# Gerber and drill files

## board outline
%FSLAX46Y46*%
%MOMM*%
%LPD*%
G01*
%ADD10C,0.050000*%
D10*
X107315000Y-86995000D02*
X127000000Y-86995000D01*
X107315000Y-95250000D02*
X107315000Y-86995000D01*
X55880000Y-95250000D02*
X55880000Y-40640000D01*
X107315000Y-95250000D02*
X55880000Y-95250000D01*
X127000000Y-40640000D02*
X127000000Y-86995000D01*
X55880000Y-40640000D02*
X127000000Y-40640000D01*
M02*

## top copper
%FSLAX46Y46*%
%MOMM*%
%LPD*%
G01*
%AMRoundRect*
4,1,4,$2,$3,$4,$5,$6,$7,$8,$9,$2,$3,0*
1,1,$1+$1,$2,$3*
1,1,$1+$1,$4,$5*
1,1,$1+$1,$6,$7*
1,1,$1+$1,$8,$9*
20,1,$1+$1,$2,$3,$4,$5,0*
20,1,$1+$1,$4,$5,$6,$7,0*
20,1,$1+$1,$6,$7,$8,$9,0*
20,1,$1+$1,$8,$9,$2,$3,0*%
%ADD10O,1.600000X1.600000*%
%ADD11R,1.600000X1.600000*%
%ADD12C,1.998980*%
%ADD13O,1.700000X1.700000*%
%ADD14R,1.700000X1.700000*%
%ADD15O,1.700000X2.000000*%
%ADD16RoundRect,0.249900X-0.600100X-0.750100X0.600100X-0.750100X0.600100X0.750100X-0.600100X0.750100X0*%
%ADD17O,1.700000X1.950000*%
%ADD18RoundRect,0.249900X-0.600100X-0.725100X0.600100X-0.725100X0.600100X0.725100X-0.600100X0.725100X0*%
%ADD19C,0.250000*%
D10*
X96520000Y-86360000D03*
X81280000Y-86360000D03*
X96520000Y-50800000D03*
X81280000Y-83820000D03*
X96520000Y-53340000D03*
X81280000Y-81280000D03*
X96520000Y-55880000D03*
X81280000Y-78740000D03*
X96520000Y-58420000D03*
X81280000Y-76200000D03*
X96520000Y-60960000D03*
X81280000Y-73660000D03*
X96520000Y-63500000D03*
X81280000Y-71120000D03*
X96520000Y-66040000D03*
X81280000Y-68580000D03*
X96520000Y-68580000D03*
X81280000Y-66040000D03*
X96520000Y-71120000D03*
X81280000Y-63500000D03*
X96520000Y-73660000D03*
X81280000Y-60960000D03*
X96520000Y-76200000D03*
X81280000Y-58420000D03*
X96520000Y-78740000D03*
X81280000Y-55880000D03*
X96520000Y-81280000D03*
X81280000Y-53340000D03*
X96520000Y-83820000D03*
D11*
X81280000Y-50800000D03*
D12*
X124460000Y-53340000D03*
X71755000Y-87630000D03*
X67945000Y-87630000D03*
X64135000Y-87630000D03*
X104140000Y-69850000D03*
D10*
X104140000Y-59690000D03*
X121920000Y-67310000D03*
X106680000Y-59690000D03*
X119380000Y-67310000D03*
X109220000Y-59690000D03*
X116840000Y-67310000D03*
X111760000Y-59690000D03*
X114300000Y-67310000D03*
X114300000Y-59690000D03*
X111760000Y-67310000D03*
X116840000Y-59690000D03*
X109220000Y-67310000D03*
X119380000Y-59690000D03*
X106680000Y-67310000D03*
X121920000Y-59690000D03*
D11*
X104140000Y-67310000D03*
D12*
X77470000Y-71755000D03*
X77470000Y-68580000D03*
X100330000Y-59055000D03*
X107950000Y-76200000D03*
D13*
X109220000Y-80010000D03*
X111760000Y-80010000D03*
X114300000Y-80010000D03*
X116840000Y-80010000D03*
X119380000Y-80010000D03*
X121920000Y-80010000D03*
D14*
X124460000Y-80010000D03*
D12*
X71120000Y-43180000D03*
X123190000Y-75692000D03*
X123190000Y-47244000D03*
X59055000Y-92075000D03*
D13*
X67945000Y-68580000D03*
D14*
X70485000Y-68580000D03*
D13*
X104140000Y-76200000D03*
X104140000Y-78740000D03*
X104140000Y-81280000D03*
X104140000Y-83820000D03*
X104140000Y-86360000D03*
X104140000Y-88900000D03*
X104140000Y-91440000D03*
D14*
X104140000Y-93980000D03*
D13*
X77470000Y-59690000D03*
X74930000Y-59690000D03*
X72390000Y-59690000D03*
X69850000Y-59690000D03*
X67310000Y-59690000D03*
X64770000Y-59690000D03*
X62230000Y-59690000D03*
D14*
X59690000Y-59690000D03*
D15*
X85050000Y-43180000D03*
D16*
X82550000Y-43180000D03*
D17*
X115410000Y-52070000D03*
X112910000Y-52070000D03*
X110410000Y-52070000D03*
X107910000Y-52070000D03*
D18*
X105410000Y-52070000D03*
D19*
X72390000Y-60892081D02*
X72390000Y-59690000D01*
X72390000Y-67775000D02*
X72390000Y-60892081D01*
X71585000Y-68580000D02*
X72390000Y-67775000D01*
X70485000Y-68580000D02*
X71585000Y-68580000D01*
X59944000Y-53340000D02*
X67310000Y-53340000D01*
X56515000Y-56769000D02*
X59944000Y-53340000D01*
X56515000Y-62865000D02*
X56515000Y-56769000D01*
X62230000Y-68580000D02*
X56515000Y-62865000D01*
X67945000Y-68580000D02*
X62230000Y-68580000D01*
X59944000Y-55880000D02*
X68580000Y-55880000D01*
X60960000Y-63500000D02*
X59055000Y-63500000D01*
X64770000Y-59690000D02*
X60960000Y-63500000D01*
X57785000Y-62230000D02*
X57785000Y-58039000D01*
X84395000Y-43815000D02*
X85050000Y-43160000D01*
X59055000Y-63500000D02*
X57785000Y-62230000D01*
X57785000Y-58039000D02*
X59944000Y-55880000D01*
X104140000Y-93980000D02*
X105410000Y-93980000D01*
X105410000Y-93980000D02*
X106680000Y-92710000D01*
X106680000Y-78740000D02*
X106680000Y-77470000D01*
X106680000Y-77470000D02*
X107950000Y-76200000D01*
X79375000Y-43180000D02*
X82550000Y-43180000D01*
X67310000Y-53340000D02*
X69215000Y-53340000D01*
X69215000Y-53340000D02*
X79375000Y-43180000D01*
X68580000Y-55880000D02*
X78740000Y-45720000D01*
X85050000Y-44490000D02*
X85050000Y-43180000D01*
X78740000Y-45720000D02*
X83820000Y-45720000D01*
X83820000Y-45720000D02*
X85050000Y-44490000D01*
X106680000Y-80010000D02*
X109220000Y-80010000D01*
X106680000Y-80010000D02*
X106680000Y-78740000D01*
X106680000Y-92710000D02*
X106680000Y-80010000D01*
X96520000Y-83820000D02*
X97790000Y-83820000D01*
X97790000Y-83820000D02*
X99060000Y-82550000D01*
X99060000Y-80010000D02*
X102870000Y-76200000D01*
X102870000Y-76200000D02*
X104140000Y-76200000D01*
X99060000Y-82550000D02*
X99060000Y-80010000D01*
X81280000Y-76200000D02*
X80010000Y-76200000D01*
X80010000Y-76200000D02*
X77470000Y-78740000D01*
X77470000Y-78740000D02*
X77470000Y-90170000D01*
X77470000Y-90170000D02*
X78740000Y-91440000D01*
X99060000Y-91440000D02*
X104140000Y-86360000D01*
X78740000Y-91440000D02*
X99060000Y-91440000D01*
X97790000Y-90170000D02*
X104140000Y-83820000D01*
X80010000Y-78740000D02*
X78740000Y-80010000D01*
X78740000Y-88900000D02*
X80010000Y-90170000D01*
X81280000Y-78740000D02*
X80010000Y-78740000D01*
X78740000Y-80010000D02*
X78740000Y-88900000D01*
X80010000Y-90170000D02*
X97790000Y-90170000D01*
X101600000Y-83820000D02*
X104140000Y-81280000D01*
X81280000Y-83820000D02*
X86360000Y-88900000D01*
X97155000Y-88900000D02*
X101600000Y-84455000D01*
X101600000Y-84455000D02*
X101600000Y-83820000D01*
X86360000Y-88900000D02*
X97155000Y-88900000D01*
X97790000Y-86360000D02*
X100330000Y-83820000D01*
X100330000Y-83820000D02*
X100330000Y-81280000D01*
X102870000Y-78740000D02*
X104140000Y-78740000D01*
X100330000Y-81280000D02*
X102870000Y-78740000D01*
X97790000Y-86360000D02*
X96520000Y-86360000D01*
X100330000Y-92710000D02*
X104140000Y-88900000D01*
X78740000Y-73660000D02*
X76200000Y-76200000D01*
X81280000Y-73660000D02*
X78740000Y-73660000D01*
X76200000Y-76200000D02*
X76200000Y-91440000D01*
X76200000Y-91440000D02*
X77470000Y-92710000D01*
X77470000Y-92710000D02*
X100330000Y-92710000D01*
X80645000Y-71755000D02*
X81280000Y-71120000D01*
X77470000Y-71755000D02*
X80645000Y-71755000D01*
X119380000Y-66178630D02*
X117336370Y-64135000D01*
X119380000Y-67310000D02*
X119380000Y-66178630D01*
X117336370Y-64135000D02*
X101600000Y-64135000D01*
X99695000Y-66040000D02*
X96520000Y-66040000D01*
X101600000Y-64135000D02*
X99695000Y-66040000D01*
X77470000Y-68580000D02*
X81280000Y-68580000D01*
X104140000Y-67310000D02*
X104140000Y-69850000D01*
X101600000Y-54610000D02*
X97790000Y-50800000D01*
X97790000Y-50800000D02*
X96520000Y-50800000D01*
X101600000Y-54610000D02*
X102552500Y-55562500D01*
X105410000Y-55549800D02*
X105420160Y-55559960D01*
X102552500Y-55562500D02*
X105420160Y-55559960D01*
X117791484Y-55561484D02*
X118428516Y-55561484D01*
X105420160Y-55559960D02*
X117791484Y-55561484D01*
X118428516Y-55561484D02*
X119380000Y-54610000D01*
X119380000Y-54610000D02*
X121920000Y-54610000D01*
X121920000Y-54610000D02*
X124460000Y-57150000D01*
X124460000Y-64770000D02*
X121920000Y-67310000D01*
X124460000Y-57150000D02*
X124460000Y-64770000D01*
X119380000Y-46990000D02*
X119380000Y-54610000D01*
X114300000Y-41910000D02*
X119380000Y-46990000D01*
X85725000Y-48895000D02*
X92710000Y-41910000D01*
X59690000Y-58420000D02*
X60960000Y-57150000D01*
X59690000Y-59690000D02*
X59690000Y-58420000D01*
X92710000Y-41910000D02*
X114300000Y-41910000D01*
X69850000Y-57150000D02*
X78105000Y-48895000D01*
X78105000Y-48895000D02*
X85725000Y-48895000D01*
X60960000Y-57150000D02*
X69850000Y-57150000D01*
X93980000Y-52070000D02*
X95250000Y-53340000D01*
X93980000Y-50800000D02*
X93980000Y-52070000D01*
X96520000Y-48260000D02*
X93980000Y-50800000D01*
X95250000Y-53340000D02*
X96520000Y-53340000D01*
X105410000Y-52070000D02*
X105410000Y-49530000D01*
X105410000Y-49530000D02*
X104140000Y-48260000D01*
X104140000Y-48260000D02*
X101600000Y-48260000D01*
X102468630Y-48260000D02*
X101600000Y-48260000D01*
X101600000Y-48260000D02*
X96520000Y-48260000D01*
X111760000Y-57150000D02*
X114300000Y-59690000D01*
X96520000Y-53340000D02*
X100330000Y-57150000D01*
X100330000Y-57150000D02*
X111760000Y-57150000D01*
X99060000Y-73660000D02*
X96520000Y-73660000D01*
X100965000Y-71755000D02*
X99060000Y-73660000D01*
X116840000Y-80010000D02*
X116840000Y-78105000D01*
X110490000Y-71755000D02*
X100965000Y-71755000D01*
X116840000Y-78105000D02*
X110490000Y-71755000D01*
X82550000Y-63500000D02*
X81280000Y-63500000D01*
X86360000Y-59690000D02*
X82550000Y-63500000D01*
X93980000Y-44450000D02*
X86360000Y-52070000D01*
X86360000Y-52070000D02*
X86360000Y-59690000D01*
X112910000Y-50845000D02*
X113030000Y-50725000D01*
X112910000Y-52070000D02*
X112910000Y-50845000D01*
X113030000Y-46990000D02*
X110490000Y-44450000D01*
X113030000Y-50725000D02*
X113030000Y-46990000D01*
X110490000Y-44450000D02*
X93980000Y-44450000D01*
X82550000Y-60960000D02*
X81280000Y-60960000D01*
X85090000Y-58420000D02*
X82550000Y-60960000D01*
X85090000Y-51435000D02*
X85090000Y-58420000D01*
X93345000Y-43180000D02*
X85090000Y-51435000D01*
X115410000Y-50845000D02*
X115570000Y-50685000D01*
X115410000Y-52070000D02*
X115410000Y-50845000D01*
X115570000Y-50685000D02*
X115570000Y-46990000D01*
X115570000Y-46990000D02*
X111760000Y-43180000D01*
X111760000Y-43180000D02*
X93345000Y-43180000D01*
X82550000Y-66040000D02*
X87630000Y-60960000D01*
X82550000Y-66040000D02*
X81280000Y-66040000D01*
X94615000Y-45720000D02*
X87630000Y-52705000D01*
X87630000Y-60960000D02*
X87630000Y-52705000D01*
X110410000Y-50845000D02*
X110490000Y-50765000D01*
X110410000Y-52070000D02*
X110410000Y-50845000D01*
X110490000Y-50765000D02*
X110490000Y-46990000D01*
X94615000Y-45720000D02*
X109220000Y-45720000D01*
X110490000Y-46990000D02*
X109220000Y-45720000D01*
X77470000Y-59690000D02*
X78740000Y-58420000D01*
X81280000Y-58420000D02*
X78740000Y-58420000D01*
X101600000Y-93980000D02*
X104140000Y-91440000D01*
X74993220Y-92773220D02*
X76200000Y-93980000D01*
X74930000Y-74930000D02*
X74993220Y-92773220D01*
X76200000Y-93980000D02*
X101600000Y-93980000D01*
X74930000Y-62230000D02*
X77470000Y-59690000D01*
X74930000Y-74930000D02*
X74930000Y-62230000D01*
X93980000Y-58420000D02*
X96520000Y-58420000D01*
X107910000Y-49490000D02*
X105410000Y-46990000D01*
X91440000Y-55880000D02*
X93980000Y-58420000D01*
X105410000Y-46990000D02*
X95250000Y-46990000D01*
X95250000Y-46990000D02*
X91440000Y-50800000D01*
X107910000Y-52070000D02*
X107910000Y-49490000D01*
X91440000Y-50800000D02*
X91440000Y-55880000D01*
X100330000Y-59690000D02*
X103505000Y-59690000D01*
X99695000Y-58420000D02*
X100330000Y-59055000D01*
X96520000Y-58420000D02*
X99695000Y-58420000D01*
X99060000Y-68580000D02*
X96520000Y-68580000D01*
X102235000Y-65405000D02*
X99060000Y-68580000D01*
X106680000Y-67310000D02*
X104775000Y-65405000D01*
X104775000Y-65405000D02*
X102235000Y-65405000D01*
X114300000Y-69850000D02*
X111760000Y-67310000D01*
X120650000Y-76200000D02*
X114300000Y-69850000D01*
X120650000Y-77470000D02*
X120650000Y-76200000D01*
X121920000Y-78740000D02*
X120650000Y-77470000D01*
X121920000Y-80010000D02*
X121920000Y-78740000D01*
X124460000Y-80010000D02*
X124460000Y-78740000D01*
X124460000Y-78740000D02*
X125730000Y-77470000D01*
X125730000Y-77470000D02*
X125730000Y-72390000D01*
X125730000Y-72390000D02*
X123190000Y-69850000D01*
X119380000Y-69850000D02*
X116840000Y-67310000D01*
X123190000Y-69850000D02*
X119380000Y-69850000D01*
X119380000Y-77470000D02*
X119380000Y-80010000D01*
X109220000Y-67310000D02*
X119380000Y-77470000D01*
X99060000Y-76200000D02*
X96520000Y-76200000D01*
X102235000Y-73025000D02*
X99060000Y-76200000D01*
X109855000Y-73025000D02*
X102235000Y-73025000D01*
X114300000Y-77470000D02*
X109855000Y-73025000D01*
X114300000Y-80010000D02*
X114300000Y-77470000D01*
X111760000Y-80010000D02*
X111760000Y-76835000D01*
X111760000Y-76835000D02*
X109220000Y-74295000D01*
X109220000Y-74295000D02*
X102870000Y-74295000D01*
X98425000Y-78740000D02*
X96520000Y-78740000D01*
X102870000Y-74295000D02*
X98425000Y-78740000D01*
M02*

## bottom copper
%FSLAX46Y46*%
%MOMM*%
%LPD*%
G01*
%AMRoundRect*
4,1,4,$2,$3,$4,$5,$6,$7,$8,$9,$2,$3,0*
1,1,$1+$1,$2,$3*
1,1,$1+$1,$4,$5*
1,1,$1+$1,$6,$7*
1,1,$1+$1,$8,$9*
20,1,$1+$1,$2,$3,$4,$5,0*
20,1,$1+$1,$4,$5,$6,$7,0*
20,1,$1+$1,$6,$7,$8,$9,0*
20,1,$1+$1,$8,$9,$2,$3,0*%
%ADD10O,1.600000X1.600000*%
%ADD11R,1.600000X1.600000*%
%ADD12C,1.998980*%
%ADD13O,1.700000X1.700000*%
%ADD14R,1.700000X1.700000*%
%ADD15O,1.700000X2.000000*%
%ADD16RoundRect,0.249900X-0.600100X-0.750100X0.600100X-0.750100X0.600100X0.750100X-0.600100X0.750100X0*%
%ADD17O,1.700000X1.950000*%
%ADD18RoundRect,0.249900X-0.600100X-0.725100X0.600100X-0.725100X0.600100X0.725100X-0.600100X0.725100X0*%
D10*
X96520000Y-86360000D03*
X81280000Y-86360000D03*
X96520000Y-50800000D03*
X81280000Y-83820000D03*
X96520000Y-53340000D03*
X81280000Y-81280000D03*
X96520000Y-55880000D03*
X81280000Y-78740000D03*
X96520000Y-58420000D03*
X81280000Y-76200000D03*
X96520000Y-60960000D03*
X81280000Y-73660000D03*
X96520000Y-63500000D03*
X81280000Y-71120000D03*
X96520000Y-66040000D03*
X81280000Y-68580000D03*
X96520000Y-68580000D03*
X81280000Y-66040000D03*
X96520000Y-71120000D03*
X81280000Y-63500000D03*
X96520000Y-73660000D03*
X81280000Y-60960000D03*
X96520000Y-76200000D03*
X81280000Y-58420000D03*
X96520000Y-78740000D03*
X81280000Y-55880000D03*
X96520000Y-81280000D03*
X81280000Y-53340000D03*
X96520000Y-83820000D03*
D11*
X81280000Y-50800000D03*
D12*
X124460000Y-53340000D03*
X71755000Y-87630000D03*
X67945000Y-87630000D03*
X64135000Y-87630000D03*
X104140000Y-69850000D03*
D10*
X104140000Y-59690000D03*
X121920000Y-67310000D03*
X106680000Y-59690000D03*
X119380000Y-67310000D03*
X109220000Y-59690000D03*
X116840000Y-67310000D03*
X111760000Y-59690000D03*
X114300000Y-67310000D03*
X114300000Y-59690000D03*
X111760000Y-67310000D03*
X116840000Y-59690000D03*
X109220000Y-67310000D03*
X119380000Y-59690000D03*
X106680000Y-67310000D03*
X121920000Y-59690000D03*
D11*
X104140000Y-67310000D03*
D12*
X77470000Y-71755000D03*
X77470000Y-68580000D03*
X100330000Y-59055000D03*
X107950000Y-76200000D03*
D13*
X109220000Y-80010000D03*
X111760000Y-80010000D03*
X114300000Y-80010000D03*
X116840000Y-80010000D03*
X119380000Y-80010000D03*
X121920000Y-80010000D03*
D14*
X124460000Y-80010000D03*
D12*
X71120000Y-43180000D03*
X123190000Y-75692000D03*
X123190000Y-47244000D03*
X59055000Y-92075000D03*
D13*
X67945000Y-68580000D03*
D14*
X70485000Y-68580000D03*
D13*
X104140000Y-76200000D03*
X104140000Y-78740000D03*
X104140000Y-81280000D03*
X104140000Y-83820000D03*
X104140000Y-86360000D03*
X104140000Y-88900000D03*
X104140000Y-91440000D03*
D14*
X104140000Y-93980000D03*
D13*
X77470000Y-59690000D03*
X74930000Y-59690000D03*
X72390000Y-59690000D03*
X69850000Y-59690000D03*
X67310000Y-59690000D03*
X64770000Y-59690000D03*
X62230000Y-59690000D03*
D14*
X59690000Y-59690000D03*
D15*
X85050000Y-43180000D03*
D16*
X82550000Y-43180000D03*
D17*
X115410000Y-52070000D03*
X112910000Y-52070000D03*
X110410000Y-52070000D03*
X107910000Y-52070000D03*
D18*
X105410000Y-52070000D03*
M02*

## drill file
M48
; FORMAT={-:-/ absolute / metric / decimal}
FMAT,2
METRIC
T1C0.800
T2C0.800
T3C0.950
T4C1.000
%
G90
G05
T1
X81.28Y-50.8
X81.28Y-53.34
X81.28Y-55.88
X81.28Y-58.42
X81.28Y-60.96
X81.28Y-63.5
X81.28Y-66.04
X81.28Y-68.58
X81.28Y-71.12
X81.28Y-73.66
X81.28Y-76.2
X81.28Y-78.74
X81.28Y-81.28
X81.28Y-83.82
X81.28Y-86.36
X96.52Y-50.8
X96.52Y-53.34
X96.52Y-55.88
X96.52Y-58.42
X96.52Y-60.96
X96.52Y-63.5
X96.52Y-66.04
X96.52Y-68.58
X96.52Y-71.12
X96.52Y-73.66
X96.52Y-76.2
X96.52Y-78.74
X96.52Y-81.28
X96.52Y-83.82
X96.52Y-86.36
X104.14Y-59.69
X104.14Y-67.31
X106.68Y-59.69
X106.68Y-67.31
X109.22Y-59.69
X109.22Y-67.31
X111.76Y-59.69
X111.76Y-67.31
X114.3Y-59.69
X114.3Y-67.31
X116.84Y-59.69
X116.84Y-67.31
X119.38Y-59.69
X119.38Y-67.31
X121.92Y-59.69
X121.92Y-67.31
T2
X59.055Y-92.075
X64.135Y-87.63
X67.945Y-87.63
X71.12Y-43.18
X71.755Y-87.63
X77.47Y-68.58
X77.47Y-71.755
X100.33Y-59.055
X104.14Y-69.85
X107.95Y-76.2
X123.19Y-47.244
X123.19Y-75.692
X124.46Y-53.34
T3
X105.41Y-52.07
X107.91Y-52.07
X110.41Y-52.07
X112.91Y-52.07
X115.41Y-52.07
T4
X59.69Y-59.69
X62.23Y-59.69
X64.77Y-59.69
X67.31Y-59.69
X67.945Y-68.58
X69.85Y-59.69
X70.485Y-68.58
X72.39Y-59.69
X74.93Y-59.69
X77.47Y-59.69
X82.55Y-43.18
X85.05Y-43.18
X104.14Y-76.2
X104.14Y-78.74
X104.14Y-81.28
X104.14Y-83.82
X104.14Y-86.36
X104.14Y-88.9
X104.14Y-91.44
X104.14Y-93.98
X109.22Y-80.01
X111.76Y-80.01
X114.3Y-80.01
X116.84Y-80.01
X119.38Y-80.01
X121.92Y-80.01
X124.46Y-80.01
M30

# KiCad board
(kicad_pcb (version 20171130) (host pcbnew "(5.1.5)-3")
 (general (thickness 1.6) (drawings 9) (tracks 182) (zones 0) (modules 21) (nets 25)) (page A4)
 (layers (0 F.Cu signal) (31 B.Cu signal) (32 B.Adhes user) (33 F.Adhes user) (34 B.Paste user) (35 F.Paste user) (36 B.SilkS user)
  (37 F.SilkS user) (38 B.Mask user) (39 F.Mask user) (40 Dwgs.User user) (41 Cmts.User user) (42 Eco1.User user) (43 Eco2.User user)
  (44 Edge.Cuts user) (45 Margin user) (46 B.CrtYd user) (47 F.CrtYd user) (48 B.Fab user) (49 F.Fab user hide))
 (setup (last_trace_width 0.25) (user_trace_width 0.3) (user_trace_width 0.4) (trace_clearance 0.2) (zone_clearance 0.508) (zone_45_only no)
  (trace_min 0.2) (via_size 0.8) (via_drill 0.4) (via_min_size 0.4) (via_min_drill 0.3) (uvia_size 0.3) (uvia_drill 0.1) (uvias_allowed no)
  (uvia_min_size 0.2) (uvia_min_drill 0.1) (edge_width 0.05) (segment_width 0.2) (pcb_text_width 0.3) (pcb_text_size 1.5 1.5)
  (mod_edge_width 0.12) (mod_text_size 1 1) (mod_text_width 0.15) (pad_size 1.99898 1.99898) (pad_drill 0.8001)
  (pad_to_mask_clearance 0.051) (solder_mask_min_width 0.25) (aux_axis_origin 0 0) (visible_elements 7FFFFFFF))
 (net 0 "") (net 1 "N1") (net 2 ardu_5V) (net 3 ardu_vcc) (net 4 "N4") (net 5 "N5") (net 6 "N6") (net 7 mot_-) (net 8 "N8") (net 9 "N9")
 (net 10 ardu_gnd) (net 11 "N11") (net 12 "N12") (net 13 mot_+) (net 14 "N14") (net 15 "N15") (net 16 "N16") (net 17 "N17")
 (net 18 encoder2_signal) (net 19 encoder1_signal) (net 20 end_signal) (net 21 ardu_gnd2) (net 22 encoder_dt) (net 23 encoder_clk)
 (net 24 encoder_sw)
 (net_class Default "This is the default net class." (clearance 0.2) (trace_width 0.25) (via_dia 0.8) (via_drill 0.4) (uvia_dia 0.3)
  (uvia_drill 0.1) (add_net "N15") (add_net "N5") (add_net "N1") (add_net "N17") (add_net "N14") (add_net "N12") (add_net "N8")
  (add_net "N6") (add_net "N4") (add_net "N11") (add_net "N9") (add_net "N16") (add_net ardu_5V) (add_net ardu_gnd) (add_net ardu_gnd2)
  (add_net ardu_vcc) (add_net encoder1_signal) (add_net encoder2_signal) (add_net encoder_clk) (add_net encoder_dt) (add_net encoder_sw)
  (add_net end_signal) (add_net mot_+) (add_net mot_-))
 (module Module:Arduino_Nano (layer F.Cu) (at 81.28 50.8)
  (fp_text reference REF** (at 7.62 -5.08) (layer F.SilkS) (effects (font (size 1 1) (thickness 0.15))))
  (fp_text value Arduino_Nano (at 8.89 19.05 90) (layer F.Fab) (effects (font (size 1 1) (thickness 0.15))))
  (pad 16 thru_hole oval (at 15.24 35.56) (size 1.6 1.6) (drill 0.8) (layers *.Cu *.Mask))
  (pad 15 thru_hole oval (at 0 35.56) (size 1.6 1.6) (drill 0.8) (layers *.Cu *.Mask))
  (pad 30 thru_hole oval (at 15.24 0) (size 1.6 1.6) (drill 0.8) (layers *.Cu *.Mask))
  (pad 14 thru_hole oval (at 0 33.02) (size 1.6 1.6) (drill 0.8) (layers *.Cu *.Mask))
  (pad 29 thru_hole oval (at 15.24 2.54) (size 1.6 1.6) (drill 0.8) (layers *.Cu *.Mask))
  (pad 13 thru_hole oval (at 0 30.48) (size 1.6 1.6) (drill 0.8) (layers *.Cu *.Mask))
  (pad 28 thru_hole oval (at 15.24 5.08) (size 1.6 1.6) (drill 0.8) (layers *.Cu *.Mask))
  (pad 12 thru_hole oval (at 0 27.94) (size 1.6 1.6) (drill 0.8) (layers *.Cu *.Mask))
  (pad 27 thru_hole oval (at 15.24 7.62) (size 1.6 1.6) (drill 0.8) (layers *.Cu *.Mask))
  (pad 11 thru_hole oval (at 0 25.4) (size 1.6 1.6) (drill 0.8) (layers *.Cu *.Mask))
  (pad 26 thru_hole oval (at 15.24 10.16) (size 1.6 1.6) (drill 0.8) (layers *.Cu *.Mask))
  (pad 10 thru_hole oval (at 0 22.86) (size 1.6 1.6) (drill 0.8) (layers *.Cu *.Mask))
  (pad 25 thru_hole oval (at 15.24 12.7) (size 1.6 1.6) (drill 0.8) (layers *.Cu *.Mask))
  (pad 9 thru_hole oval (at 0 20.32) (size 1.6 1.6) (drill 0.8) (layers *.Cu *.Mask))
  (pad 24 thru_hole oval (at 15.24 15.24) (size 1.6 1.6) (drill 0.8) (layers *.Cu *.Mask))
  (pad 8 thru_hole oval (at 0 17.78) (size 1.6 1.6) (drill 0.8) (layers *.Cu *.Mask))
  (pad 23 thru_hole oval (at 15.24 17.78) (size 1.6 1.6) (drill 0.8) (layers *.Cu *.Mask))
  (pad 7 thru_hole oval (at 0 15.24) (size 1.6 1.6) (drill 0.8) (layers *.Cu *.Mask))
  (pad 22 thru_hole oval (at 15.24 20.32) (size 1.6 1.6) (drill 0.8) (layers *.Cu *.Mask))
  (pad 6 thru_hole oval (at 0 12.7) (size 1.6 1.6) (drill 0.8) (layers *.Cu *.Mask))
  (pad 21 thru_hole oval (at 15.24 22.86) (size 1.6 1.6) (drill 0.8) (layers *.Cu *.Mask))
  (pad 5 thru_hole oval (at 0 10.16) (size 1.6 1.6) (drill 0.8) (layers *.Cu *.Mask))
  (pad 20 thru_hole oval (at 15.24 25.4) (size 1.6 1.6) (drill 0.8) (layers *.Cu *.Mask))
  (pad 4 thru_hole oval (at 0 7.62) (size 1.6 1.6) (drill 0.8) (layers *.Cu *.Mask))
  (pad 19 thru_hole oval (at 15.24 27.94) (size 1.6 1.6) (drill 0.8) (layers *.Cu *.Mask))
  (pad 3 thru_hole oval (at 0 5.08) (size 1.6 1.6) (drill 0.8) (layers *.Cu *.Mask))
  (pad 18 thru_hole oval (at 15.24 30.48) (size 1.6 1.6) (drill 0.8) (layers *.Cu *.Mask))
  (pad 2 thru_hole oval (at 0 2.54) (size 1.6 1.6) (drill 0.8) (layers *.Cu *.Mask))
  (pad 17 thru_hole oval (at 15.24 33.02) (size 1.6 1.6) (drill 0.8) (layers *.Cu *.Mask))
  (pad 1 thru_hole rect (at 0 0) (size 1.6 1.6) (drill 0.8) (layers *.Cu *.Mask)))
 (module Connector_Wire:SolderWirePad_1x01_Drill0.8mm (layer F.Cu) (at 124.46 53.34)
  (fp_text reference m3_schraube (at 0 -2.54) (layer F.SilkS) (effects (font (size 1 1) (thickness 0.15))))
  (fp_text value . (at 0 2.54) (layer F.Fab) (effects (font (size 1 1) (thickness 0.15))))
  (pad 1 thru_hole circle (at 0 0) (size 1.99898 1.99898) (drill 0.8001) (layers *.Cu *.Mask)))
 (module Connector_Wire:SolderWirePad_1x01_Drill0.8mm (layer F.Cu) (at 71.755 87.63)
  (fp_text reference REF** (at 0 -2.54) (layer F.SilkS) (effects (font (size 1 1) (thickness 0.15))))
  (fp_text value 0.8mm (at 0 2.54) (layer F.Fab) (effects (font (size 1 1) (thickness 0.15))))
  (pad 1 thru_hole circle (at 0 0) (size 1.99898 1.99898) (drill 0.8001) (layers *.Cu *.Mask)))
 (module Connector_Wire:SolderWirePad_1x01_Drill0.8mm (layer F.Cu) (at 67.945 87.63)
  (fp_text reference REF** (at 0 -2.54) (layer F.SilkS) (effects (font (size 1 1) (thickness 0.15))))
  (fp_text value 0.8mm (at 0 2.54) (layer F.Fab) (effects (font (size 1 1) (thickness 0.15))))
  (pad 1 thru_hole circle (at 0 0) (size 1.99898 1.99898) (drill 0.8001) (layers *.Cu *.Mask)))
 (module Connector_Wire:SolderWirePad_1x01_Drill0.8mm (layer F.Cu) (at 64.135 87.63)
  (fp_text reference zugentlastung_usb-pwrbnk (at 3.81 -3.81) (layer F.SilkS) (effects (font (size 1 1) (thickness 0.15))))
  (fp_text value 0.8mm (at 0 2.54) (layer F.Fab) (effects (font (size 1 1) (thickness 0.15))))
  (pad 1 thru_hole circle (at 0 0) (size 1.99898 1.99898) (drill 0.8001) (layers *.Cu *.Mask)))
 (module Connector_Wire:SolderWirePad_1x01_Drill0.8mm (layer F.Cu) (at 104.14 69.85)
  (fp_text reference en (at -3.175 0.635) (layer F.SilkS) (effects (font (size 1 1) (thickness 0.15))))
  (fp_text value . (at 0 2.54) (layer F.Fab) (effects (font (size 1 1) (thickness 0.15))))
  (pad 1 thru_hole circle (at 0 0) (size 1.99898 1.99898) (drill 0.8001) (layers *.Cu *.Mask) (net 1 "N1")))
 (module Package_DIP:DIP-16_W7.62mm (layer F.Cu) (at 104.14 67.31 90)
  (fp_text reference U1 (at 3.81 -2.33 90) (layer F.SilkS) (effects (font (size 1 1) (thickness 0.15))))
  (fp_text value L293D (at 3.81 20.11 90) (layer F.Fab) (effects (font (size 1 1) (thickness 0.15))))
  (pad 16 thru_hole oval (at 7.62 0 90) (size 1.6 1.6) (drill 0.8) (layers *.Cu *.Mask) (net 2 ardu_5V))
  (pad 8 thru_hole oval (at 0 17.78 90) (size 1.6 1.6) (drill 0.8) (layers *.Cu *.Mask) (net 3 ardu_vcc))
  (pad 15 thru_hole oval (at 7.62 2.54 90) (size 1.6 1.6) (drill 0.8) (layers *.Cu *.Mask) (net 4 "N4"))
  (pad 7 thru_hole oval (at 0 15.24 90) (size 1.6 1.6) (drill 0.8) (layers *.Cu *.Mask) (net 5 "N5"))
  (pad 14 thru_hole oval (at 7.62 5.08 90) (size 1.6 1.6) (drill 0.8) (layers *.Cu *.Mask) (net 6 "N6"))
  (pad 6 thru_hole oval (at 0 12.7 90) (size 1.6 1.6) (drill 0.8) (layers *.Cu *.Mask) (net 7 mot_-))
  (pad 13 thru_hole oval (at 7.62 7.62 90) (size 1.6 1.6) (drill 0.8) (layers *.Cu *.Mask) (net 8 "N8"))
  (pad 5 thru_hole oval (at 0 10.16 90) (size 1.6 1.6) (drill 0.8) (layers *.Cu *.Mask) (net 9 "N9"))
  (pad 12 thru_hole oval (at 7.62 10.16 90) (size 1.6 1.6) (drill 0.8) (layers *.Cu *.Mask) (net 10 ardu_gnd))
  (pad 4 thru_hole oval (at 0 7.62 90) (size 1.6 1.6) (drill 0.8) (layers *.Cu *.Mask) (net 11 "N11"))
  (pad 11 thru_hole oval (at 7.62 12.7 90) (size 1.6 1.6) (drill 0.8) (layers *.Cu *.Mask) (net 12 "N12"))
  (pad 3 thru_hole oval (at 0 5.08 90) (size 1.6 1.6) (drill 0.8) (layers *.Cu *.Mask) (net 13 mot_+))
  (pad 10 thru_hole oval (at 7.62 15.24 90) (size 1.6 1.6) (drill 0.8) (layers *.Cu *.Mask) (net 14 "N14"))
  (pad 2 thru_hole oval (at 0 2.54 90) (size 1.6 1.6) (drill 0.8) (layers *.Cu *.Mask) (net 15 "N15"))
  (pad 9 thru_hole oval (at 7.62 17.78 90) (size 1.6 1.6) (drill 0.8) (layers *.Cu *.Mask) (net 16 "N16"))
  (pad 1 thru_hole rect (at 0 0 90) (size 1.6 1.6) (drill 0.8) (layers *.Cu *.Mask) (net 1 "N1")))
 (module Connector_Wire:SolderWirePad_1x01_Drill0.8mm (layer F.Cu) (at 77.47 71.755)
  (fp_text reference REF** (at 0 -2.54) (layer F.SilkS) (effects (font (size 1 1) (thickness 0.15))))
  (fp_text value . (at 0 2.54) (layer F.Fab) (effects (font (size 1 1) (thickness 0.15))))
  (pad 1 thru_hole circle (at 0 0) (size 1.99898 1.99898) (drill 0.8001) (layers *.Cu *.Mask) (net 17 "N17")))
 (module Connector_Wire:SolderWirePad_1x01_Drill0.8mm (layer F.Cu) (at 77.47 68.58)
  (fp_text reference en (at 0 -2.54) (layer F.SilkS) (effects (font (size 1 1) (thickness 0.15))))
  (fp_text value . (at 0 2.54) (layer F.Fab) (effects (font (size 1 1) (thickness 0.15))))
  (pad 1 thru_hole circle (at 0 0) (size 1.99898 1.99898) (drill 0.8001) (layers *.Cu *.Mask) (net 1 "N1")))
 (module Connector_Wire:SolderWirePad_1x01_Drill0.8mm (layer F.Cu) (at 100.33 59.055)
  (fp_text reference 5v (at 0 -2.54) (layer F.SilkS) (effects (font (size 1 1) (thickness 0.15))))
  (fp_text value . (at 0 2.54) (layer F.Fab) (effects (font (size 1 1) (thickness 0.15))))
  (pad 1 thru_hole circle (at 0 0) (size 1.99898 1.99898) (drill 0.8001) (layers *.Cu *.Mask) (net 2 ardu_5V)))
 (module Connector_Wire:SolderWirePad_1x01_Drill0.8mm (layer F.Cu) (at 107.95 76.2)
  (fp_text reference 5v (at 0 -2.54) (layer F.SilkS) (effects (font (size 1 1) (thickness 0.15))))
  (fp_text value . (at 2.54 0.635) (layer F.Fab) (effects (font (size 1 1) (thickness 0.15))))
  (pad 1 thru_hole circle (at 0 0) (size 1.99898 1.99898) (drill 0.8001) (layers *.Cu *.Mask)))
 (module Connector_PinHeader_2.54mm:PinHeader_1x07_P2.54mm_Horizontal (layer F.Cu) (at 124.46 80.01 270)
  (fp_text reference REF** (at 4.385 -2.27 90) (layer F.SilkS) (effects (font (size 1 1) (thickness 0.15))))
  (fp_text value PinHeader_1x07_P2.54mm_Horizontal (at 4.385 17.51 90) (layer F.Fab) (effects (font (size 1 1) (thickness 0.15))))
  (pad 7 thru_hole oval (at 0 15.24 270) (size 1.7 1.7) (drill 1) (layers *.Cu *.Mask))
  (pad 6 thru_hole oval (at 0 12.7 270) (size 1.7 1.7) (drill 1) (layers *.Cu *.Mask) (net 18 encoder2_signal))
  (pad 5 thru_hole oval (at 0 10.16 270) (size 1.7 1.7) (drill 1) (layers *.Cu *.Mask) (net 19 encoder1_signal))
  (pad 4 thru_hole oval (at 0 7.62 270) (size 1.7 1.7) (drill 1) (layers *.Cu *.Mask) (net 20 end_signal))
  (pad 3 thru_hole oval (at 0 5.08 270) (size 1.7 1.7) (drill 1) (layers *.Cu *.Mask) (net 13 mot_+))
  (pad 2 thru_hole oval (at 0 2.54 270) (size 1.7 1.7) (drill 1) (layers *.Cu *.Mask) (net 11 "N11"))
  (pad 1 thru_hole rect (at 0 0 270) (size 1.7 1.7) (drill 1) (layers *.Cu *.Mask) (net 7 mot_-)))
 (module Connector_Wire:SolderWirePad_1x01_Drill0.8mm (layer F.Cu) (at 71.12 43.18)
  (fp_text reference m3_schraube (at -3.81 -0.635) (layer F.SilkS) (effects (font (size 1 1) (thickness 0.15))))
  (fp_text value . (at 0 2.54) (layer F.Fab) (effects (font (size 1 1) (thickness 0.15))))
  (pad 1 thru_hole circle (at 0 0) (size 1.99898 1.99898) (drill 0.8001) (layers *.Cu *.Mask)))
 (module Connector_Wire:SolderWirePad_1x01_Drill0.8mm (layer F.Cu) (at 123.19 75.692)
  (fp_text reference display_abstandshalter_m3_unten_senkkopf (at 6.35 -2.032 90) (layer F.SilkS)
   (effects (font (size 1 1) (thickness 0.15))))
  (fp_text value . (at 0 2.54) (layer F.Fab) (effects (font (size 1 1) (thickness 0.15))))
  (pad 1 thru_hole circle (at 0 0) (size 1.99898 1.99898) (drill 0.8001) (layers *.Cu *.Mask)))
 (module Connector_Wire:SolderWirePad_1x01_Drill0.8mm (layer F.Cu) (at 123.19 47.244)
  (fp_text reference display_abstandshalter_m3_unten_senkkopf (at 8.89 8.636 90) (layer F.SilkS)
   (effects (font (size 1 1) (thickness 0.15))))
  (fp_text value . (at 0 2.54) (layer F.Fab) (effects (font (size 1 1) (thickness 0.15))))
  (pad 1 thru_hole circle (at 0 0) (size 1.99898 1.99898) (drill 0.8001) (layers *.Cu *.Mask)))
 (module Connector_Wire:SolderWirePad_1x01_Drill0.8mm (layer F.Cu) (at 59.055 92.075)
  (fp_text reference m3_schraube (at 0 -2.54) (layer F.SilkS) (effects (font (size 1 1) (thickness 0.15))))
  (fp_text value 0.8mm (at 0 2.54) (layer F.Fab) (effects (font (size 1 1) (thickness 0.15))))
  (pad 1 thru_hole circle (at 0 0) (size 1.99898 1.99898) (drill 0.8001) (layers *.Cu *.Mask)))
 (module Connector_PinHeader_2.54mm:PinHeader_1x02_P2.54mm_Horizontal (layer F.Cu) (at 70.485 68.58 270)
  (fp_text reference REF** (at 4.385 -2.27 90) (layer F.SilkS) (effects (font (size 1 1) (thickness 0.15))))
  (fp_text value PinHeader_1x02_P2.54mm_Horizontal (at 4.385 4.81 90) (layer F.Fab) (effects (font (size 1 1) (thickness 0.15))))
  (pad 2 thru_hole oval (at 0 2.54 270) (size 1.7 1.7) (drill 1) (layers *.Cu *.Mask))
  (pad 1 thru_hole rect (at 0 0 270) (size 1.7 1.7) (drill 1) (layers *.Cu *.Mask)))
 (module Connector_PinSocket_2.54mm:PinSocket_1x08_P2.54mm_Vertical (layer F.Cu) (at 104.14 93.98 180)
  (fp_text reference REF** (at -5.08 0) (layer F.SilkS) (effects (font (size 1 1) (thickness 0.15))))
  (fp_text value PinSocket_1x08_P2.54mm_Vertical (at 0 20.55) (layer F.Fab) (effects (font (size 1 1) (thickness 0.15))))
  (pad 8 thru_hole oval (at 0 17.78 180) (size 1.7 1.7) (drill 1) (layers *.Cu *.Mask))
  (pad 7 thru_hole oval (at 0 15.24 180) (size 1.7 1.7) (drill 1) (layers *.Cu *.Mask))
  (pad 6 thru_hole oval (at 0 12.7 180) (size 1.7 1.7) (drill 1) (layers *.Cu *.Mask))
  (pad 5 thru_hole oval (at 0 10.16 180) (size 1.7 1.7) (drill 1) (layers *.Cu *.Mask))
  (pad 4 thru_hole oval (at 0 7.62 180) (size 1.7 1.7) (drill 1) (layers *.Cu *.Mask))
  (pad 3 thru_hole oval (at 0 5.08 180) (size 1.7 1.7) (drill 1) (layers *.Cu *.Mask))
  (pad 2 thru_hole oval (at 0 2.54 180) (size 1.7 1.7) (drill 1) (layers *.Cu *.Mask))
  (pad 1 thru_hole rect (at 0 0 180) (size 1.7 1.7) (drill 1) (layers *.Cu *.Mask)))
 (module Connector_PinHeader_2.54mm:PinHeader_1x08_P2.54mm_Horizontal (layer F.Cu) (at 59.69 59.69 90)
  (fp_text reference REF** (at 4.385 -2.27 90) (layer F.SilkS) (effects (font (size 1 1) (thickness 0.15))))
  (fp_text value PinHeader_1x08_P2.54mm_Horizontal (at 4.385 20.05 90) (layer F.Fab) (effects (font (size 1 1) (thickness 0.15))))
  (pad 8 thru_hole oval (at 0 17.78 90) (size 1.7 1.7) (drill 1) (layers *.Cu *.Mask) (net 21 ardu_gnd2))
  (pad 7 thru_hole oval (at 0 15.24 90) (size 1.7 1.7) (drill 1) (layers *.Cu *.Mask))
  (pad 6 thru_hole oval (at 0 12.7 90) (size 1.7 1.7) (drill 1) (layers *.Cu *.Mask))
  (pad 5 thru_hole oval (at 0 10.16 90) (size 1.7 1.7) (drill 1) (layers *.Cu *.Mask))
  (pad 4 thru_hole oval (at 0 7.62 90) (size 1.7 1.7) (drill 1) (layers *.Cu *.Mask))
  (pad 3 thru_hole oval (at 0 5.08 90) (size 1.7 1.7) (drill 1) (layers *.Cu *.Mask))
  (pad 2 thru_hole oval (at 0 2.54 90) (size 1.7 1.7) (drill 1) (layers *.Cu *.Mask))
  (pad 1 thru_hole rect (at 0 0 90) (size 1.7 1.7) (drill 1) (layers *.Cu *.Mask) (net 3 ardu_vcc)))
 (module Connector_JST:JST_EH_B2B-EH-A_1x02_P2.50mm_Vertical (layer F.Cu) (at 82.55 43.18)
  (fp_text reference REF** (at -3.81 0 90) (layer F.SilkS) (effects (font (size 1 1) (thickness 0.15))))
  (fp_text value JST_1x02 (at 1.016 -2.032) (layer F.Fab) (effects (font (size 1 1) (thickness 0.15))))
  (pad 2 thru_hole oval (at 2.5 0) (size 1.7 2) (drill 1) (layers *.Cu *.Mask))
  (pad 1 thru_hole roundrect (at 0 0) (size 1.7 2) (drill 1) (layers *.Cu *.Mask) (roundrect_rratio 0.147)))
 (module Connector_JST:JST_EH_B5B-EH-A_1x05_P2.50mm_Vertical (layer F.Cu) (at 105.41 52.07)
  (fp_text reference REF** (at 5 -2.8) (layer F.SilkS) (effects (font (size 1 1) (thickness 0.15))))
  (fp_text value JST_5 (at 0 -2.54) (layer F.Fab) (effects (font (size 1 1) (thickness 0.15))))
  (pad 5 thru_hole oval (at 10 0) (size 1.7 1.95) (drill 0.95) (layers *.Cu *.Mask) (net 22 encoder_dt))
  (pad 4 thru_hole oval (at 7.5 0) (size 1.7 1.95) (drill 0.95) (layers *.Cu *.Mask) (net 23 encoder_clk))
  (pad 3 thru_hole oval (at 5 0) (size 1.7 1.95) (drill 0.95) (layers *.Cu *.Mask) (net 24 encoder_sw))
  (pad 2 thru_hole oval (at 2.5 0) (size 1.7 1.95) (drill 0.95) (layers *.Cu *.Mask) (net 2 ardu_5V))
  (pad 1 thru_hole roundrect (at 0 0) (size 1.7 1.95) (drill 0.95) (layers *.Cu *.Mask) (roundrect_rratio 0.147) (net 10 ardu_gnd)))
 (gr_line (start 107.315 86.995) (end 127 86.995) (layer Edge.Cuts) (width 0.05))
 (gr_line (start 107.315 95.25) (end 107.315 86.995) (layer Edge.Cuts) (width 0.05))
 (gr_line (start 55.88 95.25) (end 55.88 40.64) (layer Edge.Cuts) (width 0.05))
 (gr_line (start 107.315 95.25) (end 55.88 95.25) (layer Edge.Cuts) (width 0.05))
 (gr_line (start 127 40.64) (end 127 86.995) (layer Edge.Cuts) (width 0.05))
 (gr_line (start 55.88 40.64) (end 127 40.64) (layer Edge.Cuts) (width 0.05))
 (segment (start 72.39 60.892081) (end 72.39 59.69) (width 0.25) (layer F.Cu) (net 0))
 (segment (start 72.39 67.775) (end 72.39 60.892081) (width 0.25) (layer F.Cu) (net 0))
 (segment (start 71.585 68.58) (end 72.39 67.775) (width 0.25) (layer F.Cu) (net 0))
 (segment (start 70.485 68.58) (end 71.585 68.58) (width 0.25) (layer F.Cu) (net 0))
 (segment (start 59.944 53.34) (end 67.31 53.34) (width 0.25) (layer F.Cu) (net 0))
 (segment (start 56.515 56.769) (end 59.944 53.34) (width 0.25) (layer F.Cu) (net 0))
 (segment (start 56.515 62.865) (end 56.515 56.769) (width 0.25) (layer F.Cu) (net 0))
 (segment (start 62.23 68.58) (end 56.515 62.865) (width 0.25) (layer F.Cu) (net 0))
 (segment (start 67.945 68.58) (end 62.23 68.58) (width 0.25) (layer F.Cu) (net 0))
 (segment (start 59.944 55.88) (end 68.58 55.88) (width 0.25) (layer F.Cu) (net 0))
 (segment (start 60.96 63.5) (end 59.055 63.5) (width 0.25) (layer F.Cu) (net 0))
 (segment (start 64.77 59.69) (end 60.96 63.5) (width 0.25) (layer F.Cu) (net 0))
 (segment (start 57.785 62.23) (end 57.785 58.039) (width 0.25) (layer F.Cu) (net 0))
 (segment (start 84.395 43.815) (end 85.05 43.16) (width 0.25) (layer F.Cu) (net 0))
 (segment (start 59.055 63.5) (end 57.785 62.23) (width 0.25) (layer F.Cu) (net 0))
 (segment (start 57.785 58.039) (end 59.944 55.88) (width 0.25) (layer F.Cu) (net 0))
 (segment (start 104.14 93.98) (end 105.41 93.98) (width 0.25) (layer F.Cu) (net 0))
 (segment (start 105.41 93.98) (end 106.68 92.71) (width 0.25) (layer F.Cu) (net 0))
 (segment (start 106.68 78.74) (end 106.68 77.47) (width 0.25) (layer F.Cu) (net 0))
 (segment (start 106.68 77.47) (end 107.95 76.2) (width 0.25) (layer F.Cu) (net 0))
 (segment (start 79.375 43.18) (end 82.55 43.18) (width 0.25) (layer F.Cu) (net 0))
 (segment (start 67.31 53.34) (end 69.215 53.34) (width 0.25) (layer F.Cu) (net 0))
 (segment (start 69.215 53.34) (end 79.375 43.18) (width 0.25) (layer F.Cu) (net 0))
 (segment (start 68.58 55.88) (end 78.74 45.72) (width 0.25) (layer F.Cu) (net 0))
 (segment (start 85.05 44.49) (end 85.05 43.18) (width 0.25) (layer F.Cu) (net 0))
 (segment (start 78.74 45.72) (end 83.82 45.72) (width 0.25) (layer F.Cu) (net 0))
 (segment (start 83.82 45.72) (end 85.05 44.49) (width 0.25) (layer F.Cu) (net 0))
 (segment (start 106.68 80.01) (end 109.22 80.01) (width 0.25) (layer F.Cu) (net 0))
 (segment (start 106.68 80.01) (end 106.68 78.74) (width 0.25) (layer F.Cu) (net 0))
 (segment (start 106.68 92.71) (end 106.68 80.01) (width 0.25) (layer F.Cu) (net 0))
 (segment (start 96.52 83.82) (end 97.79 83.82) (width 0.25) (layer F.Cu) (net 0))
 (segment (start 97.79 83.82) (end 99.06 82.55) (width 0.25) (layer F.Cu) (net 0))
 (segment (start 99.06 80.01) (end 102.87 76.2) (width 0.25) (layer F.Cu) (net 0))
 (segment (start 102.87 76.2) (end 104.14 76.2) (width 0.25) (layer F.Cu) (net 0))
 (segment (start 99.06 82.55) (end 99.06 80.01) (width 0.25) (layer F.Cu) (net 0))
 (segment (start 81.28 76.2) (end 80.01 76.2) (width 0.25) (layer F.Cu) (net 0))
 (segment (start 80.01 76.2) (end 77.47 78.74) (width 0.25) (layer F.Cu) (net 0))
 (segment (start 77.47 78.74) (end 77.47 90.17) (width 0.25) (layer F.Cu) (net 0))
 (segment (start 77.47 90.17) (end 78.74 91.44) (width 0.25) (layer F.Cu) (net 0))
 (segment (start 99.06 91.44) (end 104.14 86.36) (width 0.25) (layer F.Cu) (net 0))
 (segment (start 78.74 91.44) (end 99.06 91.44) (width 0.25) (layer F.Cu) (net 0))
 (segment (start 97.79 90.17) (end 104.14 83.82) (width 0.25) (layer F.Cu) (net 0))
 (segment (start 80.01 78.74) (end 78.74 80.01) (width 0.25) (layer F.Cu) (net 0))
 (segment (start 78.74 88.9) (end 80.01 90.17) (width 0.25) (layer F.Cu) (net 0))
 (segment (start 81.28 78.74) (end 80.01 78.74) (width 0.25) (layer F.Cu) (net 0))
 (segment (start 78.74 80.01) (end 78.74 88.9) (width 0.25) (layer F.Cu) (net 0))
 (segment (start 80.01 90.17) (end 97.79 90.17) (width 0.25) (layer F.Cu) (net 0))
 (segment (start 101.6 83.82) (end 104.14 81.28) (width 0.25) (layer F.Cu) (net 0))
 (segment (start 81.28 83.82) (end 86.36 88.9) (width 0.25) (layer F.Cu) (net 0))
 (segment (start 97.155 88.9) (end 101.6 84.455) (width 0.25) (layer F.Cu) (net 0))
 (segment (start 101.6 84.455) (end 101.6 83.82) (width 0.25) (layer F.Cu) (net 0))
 (segment (start 86.36 88.9) (end 97.155 88.9) (width 0.25) (layer F.Cu) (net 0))
 (segment (start 97.79 86.36) (end 100.33 83.82) (width 0.25) (layer F.Cu) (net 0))
 (segment (start 100.33 83.82) (end 100.33 81.28) (width 0.25) (layer F.Cu) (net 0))
 (segment (start 102.87 78.74) (end 104.14 78.74) (width 0.25) (layer F.Cu) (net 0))
 (segment (start 100.33 81.28) (end 102.87 78.74) (width 0.25) (layer F.Cu) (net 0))
 (segment (start 97.79 86.36) (end 96.52 86.36) (width 0.25) (layer F.Cu) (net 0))
 (segment (start 100.33 92.71) (end 104.14 88.9) (width 0.25) (layer F.Cu) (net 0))
 (segment (start 78.74 73.66) (end 76.2 76.2) (width 0.25) (layer F.Cu) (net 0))
 (segment (start 81.28 73.66) (end 78.74 73.66) (width 0.25) (layer F.Cu) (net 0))
 (segment (start 76.2 76.2) (end 76.2 91.44) (width 0.25) (layer F.Cu) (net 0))
 (segment (start 76.2 91.44) (end 77.47 92.71) (width 0.25) (layer F.Cu) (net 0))
 (segment (start 77.47 92.71) (end 100.33 92.71) (width 0.25) (layer F.Cu) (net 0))
 (segment (start 80.645 71.755) (end 81.28 71.12) (width 0.25) (layer F.Cu) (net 17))
 (segment (start 77.47 71.755) (end 80.645 71.755) (width 0.25) (layer F.Cu) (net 17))
 (segment (start 119.38 66.17863) (end 117.33637 64.135) (width 0.25) (layer F.Cu) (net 5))
 (segment (start 119.38 67.31) (end 119.38 66.17863) (width 0.25) (layer F.Cu) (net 5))
 (segment (start 117.33637 64.135) (end 101.6 64.135) (width 0.25) (layer F.Cu) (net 5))
 (segment (start 99.695 66.04) (end 96.52 66.04) (width 0.25) (layer F.Cu) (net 5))
 (segment (start 101.6 64.135) (end 99.695 66.04) (width 0.25) (layer F.Cu) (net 5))
 (segment (start 77.47 68.58) (end 81.28 68.58) (width 0.25) (layer F.Cu) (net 1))
 (segment (start 104.14 67.31) (end 104.14 69.85) (width 0.25) (layer F.Cu) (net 1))
 (segment (start 101.6 54.61) (end 97.79 50.8) (width 0.25) (layer F.Cu) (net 3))
 (segment (start 97.79 50.8) (end 96.52 50.8) (width 0.25) (layer F.Cu) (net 3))
 (segment (start 101.6 54.61) (end 102.5525 55.5625) (width 0.25) (layer F.Cu) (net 3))
 (segment (start 105.41 55.5498) (end 105.42016 55.55996) (width 0.25) (layer F.Cu) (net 3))
 (segment (start 102.5525 55.5625) (end 105.42016 55.55996) (width 0.25) (layer F.Cu) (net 3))
 (segment (start 117.791484 55.561484) (end 118.428516 55.561484) (width 0.25) (layer F.Cu) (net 3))
 (segment (start 105.42016 55.55996) (end 117.791484 55.561484) (width 0.25) (layer F.Cu) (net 3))
 (segment (start 118.428516 55.561484) (end 119.38 54.61) (width 0.25) (layer F.Cu) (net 3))
 (segment (start 119.38 54.61) (end 121.92 54.61) (width 0.25) (layer F.Cu) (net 3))
 (segment (start 121.92 54.61) (end 124.46 57.15) (width 0.25) (layer F.Cu) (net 3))
 (segment (start 124.46 64.77) (end 121.92 67.31) (width 0.25) (layer F.Cu) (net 3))
 (segment (start 124.46 57.15) (end 124.46 64.77) (width 0.25) (layer F.Cu) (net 3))
 (segment (start 119.38 46.99) (end 119.38 54.61) (width 0.25) (layer F.Cu) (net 3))
 (segment (start 114.3 41.91) (end 119.38 46.99) (width 0.25) (layer F.Cu) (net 3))
 (segment (start 85.725 48.895) (end 92.71 41.91) (width 0.25) (layer F.Cu) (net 3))
 (segment (start 59.69 58.42) (end 60.96 57.15) (width 0.25) (layer F.Cu) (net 3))
 (segment (start 59.69 59.69) (end 59.69 58.42) (width 0.25) (layer F.Cu) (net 3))
 (segment (start 92.71 41.91) (end 114.3 41.91) (width 0.25) (layer F.Cu) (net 3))
 (segment (start 69.85 57.15) (end 78.105 48.895) (width 0.25) (layer F.Cu) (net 3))
 (segment (start 78.105 48.895) (end 85.725 48.895) (width 0.25) (layer F.Cu) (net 3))
 (segment (start 60.96 57.15) (end 69.85 57.15) (width 0.25) (layer F.Cu) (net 3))
 (segment (start 93.98 52.07) (end 95.25 53.34) (width 0.25) (layer F.Cu) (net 10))
 (segment (start 93.98 50.8) (end 93.98 52.07) (width 0.25) (layer F.Cu) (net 10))
 (segment (start 96.52 48.26) (end 93.98 50.8) (width 0.25) (layer F.Cu) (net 10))
 (segment (start 95.25 53.34) (end 96.52 53.34) (width 0.25) (layer F.Cu) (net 10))
 (segment (start 105.41 52.07) (end 105.41 49.53) (width 0.25) (layer F.Cu) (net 10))
 (segment (start 105.41 49.53) (end 104.14 48.26) (width 0.25) (layer F.Cu) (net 10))
 (segment (start 104.14 48.26) (end 101.6 48.26) (width 0.25) (layer F.Cu) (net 10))
 (segment (start 102.46863 48.26) (end 101.6 48.26) (width 0.25) (layer F.Cu) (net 10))
 (segment (start 101.6 48.26) (end 96.52 48.26) (width 0.25) (layer F.Cu) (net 10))
 (segment (start 111.76 57.15) (end 114.3 59.69) (width 0.25) (layer F.Cu) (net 10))
 (segment (start 96.52 53.34) (end 100.33 57.15) (width 0.25) (layer F.Cu) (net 10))
 (segment (start 100.33 57.15) (end 111.76 57.15) (width 0.25) (layer F.Cu) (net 10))
 (segment (start 99.06 73.66) (end 96.52 73.66) (width 0.25) (layer F.Cu) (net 20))
 (segment (start 100.965 71.755) (end 99.06 73.66) (width 0.25) (layer F.Cu) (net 20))
 (segment (start 116.84 80.01) (end 116.84 78.105) (width 0.25) (layer F.Cu) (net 20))
 (segment (start 110.49 71.755) (end 100.965 71.755) (width 0.25) (layer F.Cu) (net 20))
 (segment (start 116.84 78.105) (end 110.49 71.755) (width 0.25) (layer F.Cu) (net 20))
 (segment (start 82.55 63.5) (end 81.28 63.5) (width 0.25) (layer F.Cu) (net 23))
 (segment (start 86.36 59.69) (end 82.55 63.5) (width 0.25) (layer F.Cu) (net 23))
 (segment (start 93.98 44.45) (end 86.36 52.07) (width 0.25) (layer F.Cu) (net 23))
 (segment (start 86.36 52.07) (end 86.36 59.69) (width 0.25) (layer F.Cu) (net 23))
 (segment (start 112.91 50.845) (end 113.03 50.725) (width 0.25) (layer F.Cu) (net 23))
 (segment (start 112.91 52.07) (end 112.91 50.845) (width 0.25) (layer F.Cu) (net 23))
 (segment (start 113.03 46.99) (end 110.49 44.45) (width 0.25) (layer F.Cu) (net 23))
 (segment (start 113.03 50.725) (end 113.03 46.99) (width 0.25) (layer F.Cu) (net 23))
 (segment (start 110.49 44.45) (end 93.98 44.45) (width 0.25) (layer F.Cu) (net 23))
 (segment (start 82.55 60.96) (end 81.28 60.96) (width 0.25) (layer F.Cu) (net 22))
 (segment (start 85.09 58.42) (end 82.55 60.96) (width 0.25) (layer F.Cu) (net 22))
 (segment (start 85.09 51.435) (end 85.09 58.42) (width 0.25) (layer F.Cu) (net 22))
 (segment (start 93.345 43.18) (end 85.09 51.435) (width 0.25) (layer F.Cu) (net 22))
 (segment (start 115.41 50.845) (end 115.57 50.685) (width 0.25) (layer F.Cu) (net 22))
 (segment (start 115.41 52.07) (end 115.41 50.845) (width 0.25) (layer F.Cu) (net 22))
 (segment (start 115.57 50.685) (end 115.57 46.99) (width 0.25) (layer F.Cu) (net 22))
 (segment (start 115.57 46.99) (end 111.76 43.18) (width 0.25) (layer F.Cu) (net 22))
 (segment (start 111.76 43.18) (end 93.345 43.18) (width 0.25) (layer F.Cu) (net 22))
 (segment (start 82.55 66.04) (end 87.63 60.96) (width 0.25) (layer F.Cu) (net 24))
 (segment (start 82.55 66.04) (end 81.28 66.04) (width 0.25) (layer F.Cu) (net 24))
 (segment (start 94.615 45.72) (end 87.63 52.705) (width 0.25) (layer F.Cu) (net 24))
 (segment (start 87.63 60.96) (end 87.63 52.705) (width 0.25) (layer F.Cu) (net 24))
 (segment (start 110.41 50.845) (end 110.49 50.765) (width 0.25) (layer F.Cu) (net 24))
 (segment (start 110.41 52.07) (end 110.41 50.845) (width 0.25) (layer F.Cu) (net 24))
 (segment (start 110.49 50.765) (end 110.49 46.99) (width 0.25) (layer F.Cu) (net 24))
 (segment (start 94.615 45.72) (end 109.22 45.72) (width 0.25) (layer F.Cu) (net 24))
 (segment (start 110.49 46.99) (end 109.22 45.72) (width 0.25) (layer F.Cu) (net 24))
 (segment (start 77.47 59.69) (end 78.74 58.42) (width 0.25) (layer F.Cu) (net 21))
 (segment (start 81.28 58.42) (end 78.74 58.42) (width 0.25) (layer F.Cu) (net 21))
 (segment (start 101.6 93.98) (end 104.14 91.44) (width 0.25) (layer F.Cu) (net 21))
 (segment (start 74.99322 92.77322) (end 76.2 93.98) (width 0.25) (layer F.Cu) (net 21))
 (segment (start 74.93 74.93) (end 74.99322 92.77322) (width 0.25) (layer F.Cu) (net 21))
 (segment (start 76.2 93.98) (end 101.6 93.98) (width 0.25) (layer F.Cu) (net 21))
 (segment (start 74.93 62.23) (end 77.47 59.69) (width 0.25) (layer F.Cu) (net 21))
 (segment (start 74.93 74.93) (end 74.93 62.23) (width 0.25) (layer F.Cu) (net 21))
 (segment (start 93.98 58.42) (end 96.52 58.42) (width 0.25) (layer F.Cu) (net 2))
 (segment (start 107.91 49.49) (end 105.41 46.99) (width 0.25) (layer F.Cu) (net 2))
 (segment (start 91.44 55.88) (end 93.98 58.42) (width 0.25) (layer F.Cu) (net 2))
 (segment (start 105.41 46.99) (end 95.25 46.99) (width 0.25) (layer F.Cu) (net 2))
 (segment (start 95.25 46.99) (end 91.44 50.8) (width 0.25) (layer F.Cu) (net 2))
 (segment (start 107.91 52.07) (end 107.91 49.49) (width 0.25) (layer F.Cu) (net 2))
 (segment (start 91.44 50.8) (end 91.44 55.88) (width 0.25) (layer F.Cu) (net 2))
 (segment (start 100.33 59.69) (end 103.505 59.69) (width 0.25) (layer F.Cu) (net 2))
 (segment (start 99.695 58.42) (end 100.33 59.055) (width 0.25) (layer F.Cu) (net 2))
 (segment (start 96.52 58.42) (end 99.695 58.42) (width 0.25) (layer F.Cu) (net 2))
 (segment (start 99.06 68.58) (end 96.52 68.58) (width 0.25) (layer F.Cu) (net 15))
 (segment (start 102.235 65.405) (end 99.06 68.58) (width 0.25) (layer F.Cu) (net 15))
 (segment (start 106.68 67.31) (end 104.775 65.405) (width 0.25) (layer F.Cu) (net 15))
 (segment (start 104.775 65.405) (end 102.235 65.405) (width 0.25) (layer F.Cu) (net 15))
 (segment (start 114.3 69.85) (end 111.76 67.31) (width 0.25) (layer F.Cu) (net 11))
 (segment (start 120.65 76.2) (end 114.3 69.85) (width 0.25) (layer F.Cu) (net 11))
 (segment (start 120.65 77.47) (end 120.65 76.2) (width 0.25) (layer F.Cu) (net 11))
 (segment (start 121.92 78.74) (end 120.65 77.47) (width 0.25) (layer F.Cu) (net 11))
 (segment (start 121.92 80.01) (end 121.92 78.74) (width 0.25) (layer F.Cu) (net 11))
 (segment (start 124.46 80.01) (end 124.46 78.74) (width 0.25) (layer F.Cu) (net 7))
 (segment (start 124.46 78.74) (end 125.73 77.47) (width 0.25) (layer F.Cu) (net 7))
 (segment (start 125.73 77.47) (end 125.73 72.39) (width 0.25) (layer F.Cu) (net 7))
 (segment (start 125.73 72.39) (end 123.19 69.85) (width 0.25) (layer F.Cu) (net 7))
 (segment (start 119.38 69.85) (end 116.84 67.31) (width 0.25) (layer F.Cu) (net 7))
 (segment (start 123.19 69.85) (end 119.38 69.85) (width 0.25) (layer F.Cu) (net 7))
 (segment (start 119.38 77.47) (end 119.38 80.01) (width 0.25) (layer F.Cu) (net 13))
 (segment (start 109.22 67.31) (end 119.38 77.47) (width 0.25) (layer F.Cu) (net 13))
 (segment (start 99.06 76.2) (end 96.52 76.2) (width 0.25) (layer F.Cu) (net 19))
 (segment (start 102.235 73.025) (end 99.06 76.2) (width 0.25) (layer F.Cu) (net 19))
 (segment (start 109.855 73.025) (end 102.235 73.025) (width 0.25) (layer F.Cu) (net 19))
 (segment (start 114.3 77.47) (end 109.855 73.025) (width 0.25) (layer F.Cu) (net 19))
 (segment (start 114.3 80.01) (end 114.3 77.47) (width 0.25) (layer F.Cu) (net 19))
 (segment (start 111.76 80.01) (end 111.76 76.835) (width 0.25) (layer F.Cu) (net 18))
 (segment (start 111.76 76.835) (end 109.22 74.295) (width 0.25) (layer F.Cu) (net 18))
 (segment (start 109.22 74.295) (end 102.87 74.295) (width 0.25) (layer F.Cu) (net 18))
 (segment (start 98.425 78.74) (end 96.52 78.74) (width 0.25) (layer F.Cu) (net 18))
 (segment (start 102.87 74.295) (end 98.425 78.74) (width 0.25) (layer F.Cu) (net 18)))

